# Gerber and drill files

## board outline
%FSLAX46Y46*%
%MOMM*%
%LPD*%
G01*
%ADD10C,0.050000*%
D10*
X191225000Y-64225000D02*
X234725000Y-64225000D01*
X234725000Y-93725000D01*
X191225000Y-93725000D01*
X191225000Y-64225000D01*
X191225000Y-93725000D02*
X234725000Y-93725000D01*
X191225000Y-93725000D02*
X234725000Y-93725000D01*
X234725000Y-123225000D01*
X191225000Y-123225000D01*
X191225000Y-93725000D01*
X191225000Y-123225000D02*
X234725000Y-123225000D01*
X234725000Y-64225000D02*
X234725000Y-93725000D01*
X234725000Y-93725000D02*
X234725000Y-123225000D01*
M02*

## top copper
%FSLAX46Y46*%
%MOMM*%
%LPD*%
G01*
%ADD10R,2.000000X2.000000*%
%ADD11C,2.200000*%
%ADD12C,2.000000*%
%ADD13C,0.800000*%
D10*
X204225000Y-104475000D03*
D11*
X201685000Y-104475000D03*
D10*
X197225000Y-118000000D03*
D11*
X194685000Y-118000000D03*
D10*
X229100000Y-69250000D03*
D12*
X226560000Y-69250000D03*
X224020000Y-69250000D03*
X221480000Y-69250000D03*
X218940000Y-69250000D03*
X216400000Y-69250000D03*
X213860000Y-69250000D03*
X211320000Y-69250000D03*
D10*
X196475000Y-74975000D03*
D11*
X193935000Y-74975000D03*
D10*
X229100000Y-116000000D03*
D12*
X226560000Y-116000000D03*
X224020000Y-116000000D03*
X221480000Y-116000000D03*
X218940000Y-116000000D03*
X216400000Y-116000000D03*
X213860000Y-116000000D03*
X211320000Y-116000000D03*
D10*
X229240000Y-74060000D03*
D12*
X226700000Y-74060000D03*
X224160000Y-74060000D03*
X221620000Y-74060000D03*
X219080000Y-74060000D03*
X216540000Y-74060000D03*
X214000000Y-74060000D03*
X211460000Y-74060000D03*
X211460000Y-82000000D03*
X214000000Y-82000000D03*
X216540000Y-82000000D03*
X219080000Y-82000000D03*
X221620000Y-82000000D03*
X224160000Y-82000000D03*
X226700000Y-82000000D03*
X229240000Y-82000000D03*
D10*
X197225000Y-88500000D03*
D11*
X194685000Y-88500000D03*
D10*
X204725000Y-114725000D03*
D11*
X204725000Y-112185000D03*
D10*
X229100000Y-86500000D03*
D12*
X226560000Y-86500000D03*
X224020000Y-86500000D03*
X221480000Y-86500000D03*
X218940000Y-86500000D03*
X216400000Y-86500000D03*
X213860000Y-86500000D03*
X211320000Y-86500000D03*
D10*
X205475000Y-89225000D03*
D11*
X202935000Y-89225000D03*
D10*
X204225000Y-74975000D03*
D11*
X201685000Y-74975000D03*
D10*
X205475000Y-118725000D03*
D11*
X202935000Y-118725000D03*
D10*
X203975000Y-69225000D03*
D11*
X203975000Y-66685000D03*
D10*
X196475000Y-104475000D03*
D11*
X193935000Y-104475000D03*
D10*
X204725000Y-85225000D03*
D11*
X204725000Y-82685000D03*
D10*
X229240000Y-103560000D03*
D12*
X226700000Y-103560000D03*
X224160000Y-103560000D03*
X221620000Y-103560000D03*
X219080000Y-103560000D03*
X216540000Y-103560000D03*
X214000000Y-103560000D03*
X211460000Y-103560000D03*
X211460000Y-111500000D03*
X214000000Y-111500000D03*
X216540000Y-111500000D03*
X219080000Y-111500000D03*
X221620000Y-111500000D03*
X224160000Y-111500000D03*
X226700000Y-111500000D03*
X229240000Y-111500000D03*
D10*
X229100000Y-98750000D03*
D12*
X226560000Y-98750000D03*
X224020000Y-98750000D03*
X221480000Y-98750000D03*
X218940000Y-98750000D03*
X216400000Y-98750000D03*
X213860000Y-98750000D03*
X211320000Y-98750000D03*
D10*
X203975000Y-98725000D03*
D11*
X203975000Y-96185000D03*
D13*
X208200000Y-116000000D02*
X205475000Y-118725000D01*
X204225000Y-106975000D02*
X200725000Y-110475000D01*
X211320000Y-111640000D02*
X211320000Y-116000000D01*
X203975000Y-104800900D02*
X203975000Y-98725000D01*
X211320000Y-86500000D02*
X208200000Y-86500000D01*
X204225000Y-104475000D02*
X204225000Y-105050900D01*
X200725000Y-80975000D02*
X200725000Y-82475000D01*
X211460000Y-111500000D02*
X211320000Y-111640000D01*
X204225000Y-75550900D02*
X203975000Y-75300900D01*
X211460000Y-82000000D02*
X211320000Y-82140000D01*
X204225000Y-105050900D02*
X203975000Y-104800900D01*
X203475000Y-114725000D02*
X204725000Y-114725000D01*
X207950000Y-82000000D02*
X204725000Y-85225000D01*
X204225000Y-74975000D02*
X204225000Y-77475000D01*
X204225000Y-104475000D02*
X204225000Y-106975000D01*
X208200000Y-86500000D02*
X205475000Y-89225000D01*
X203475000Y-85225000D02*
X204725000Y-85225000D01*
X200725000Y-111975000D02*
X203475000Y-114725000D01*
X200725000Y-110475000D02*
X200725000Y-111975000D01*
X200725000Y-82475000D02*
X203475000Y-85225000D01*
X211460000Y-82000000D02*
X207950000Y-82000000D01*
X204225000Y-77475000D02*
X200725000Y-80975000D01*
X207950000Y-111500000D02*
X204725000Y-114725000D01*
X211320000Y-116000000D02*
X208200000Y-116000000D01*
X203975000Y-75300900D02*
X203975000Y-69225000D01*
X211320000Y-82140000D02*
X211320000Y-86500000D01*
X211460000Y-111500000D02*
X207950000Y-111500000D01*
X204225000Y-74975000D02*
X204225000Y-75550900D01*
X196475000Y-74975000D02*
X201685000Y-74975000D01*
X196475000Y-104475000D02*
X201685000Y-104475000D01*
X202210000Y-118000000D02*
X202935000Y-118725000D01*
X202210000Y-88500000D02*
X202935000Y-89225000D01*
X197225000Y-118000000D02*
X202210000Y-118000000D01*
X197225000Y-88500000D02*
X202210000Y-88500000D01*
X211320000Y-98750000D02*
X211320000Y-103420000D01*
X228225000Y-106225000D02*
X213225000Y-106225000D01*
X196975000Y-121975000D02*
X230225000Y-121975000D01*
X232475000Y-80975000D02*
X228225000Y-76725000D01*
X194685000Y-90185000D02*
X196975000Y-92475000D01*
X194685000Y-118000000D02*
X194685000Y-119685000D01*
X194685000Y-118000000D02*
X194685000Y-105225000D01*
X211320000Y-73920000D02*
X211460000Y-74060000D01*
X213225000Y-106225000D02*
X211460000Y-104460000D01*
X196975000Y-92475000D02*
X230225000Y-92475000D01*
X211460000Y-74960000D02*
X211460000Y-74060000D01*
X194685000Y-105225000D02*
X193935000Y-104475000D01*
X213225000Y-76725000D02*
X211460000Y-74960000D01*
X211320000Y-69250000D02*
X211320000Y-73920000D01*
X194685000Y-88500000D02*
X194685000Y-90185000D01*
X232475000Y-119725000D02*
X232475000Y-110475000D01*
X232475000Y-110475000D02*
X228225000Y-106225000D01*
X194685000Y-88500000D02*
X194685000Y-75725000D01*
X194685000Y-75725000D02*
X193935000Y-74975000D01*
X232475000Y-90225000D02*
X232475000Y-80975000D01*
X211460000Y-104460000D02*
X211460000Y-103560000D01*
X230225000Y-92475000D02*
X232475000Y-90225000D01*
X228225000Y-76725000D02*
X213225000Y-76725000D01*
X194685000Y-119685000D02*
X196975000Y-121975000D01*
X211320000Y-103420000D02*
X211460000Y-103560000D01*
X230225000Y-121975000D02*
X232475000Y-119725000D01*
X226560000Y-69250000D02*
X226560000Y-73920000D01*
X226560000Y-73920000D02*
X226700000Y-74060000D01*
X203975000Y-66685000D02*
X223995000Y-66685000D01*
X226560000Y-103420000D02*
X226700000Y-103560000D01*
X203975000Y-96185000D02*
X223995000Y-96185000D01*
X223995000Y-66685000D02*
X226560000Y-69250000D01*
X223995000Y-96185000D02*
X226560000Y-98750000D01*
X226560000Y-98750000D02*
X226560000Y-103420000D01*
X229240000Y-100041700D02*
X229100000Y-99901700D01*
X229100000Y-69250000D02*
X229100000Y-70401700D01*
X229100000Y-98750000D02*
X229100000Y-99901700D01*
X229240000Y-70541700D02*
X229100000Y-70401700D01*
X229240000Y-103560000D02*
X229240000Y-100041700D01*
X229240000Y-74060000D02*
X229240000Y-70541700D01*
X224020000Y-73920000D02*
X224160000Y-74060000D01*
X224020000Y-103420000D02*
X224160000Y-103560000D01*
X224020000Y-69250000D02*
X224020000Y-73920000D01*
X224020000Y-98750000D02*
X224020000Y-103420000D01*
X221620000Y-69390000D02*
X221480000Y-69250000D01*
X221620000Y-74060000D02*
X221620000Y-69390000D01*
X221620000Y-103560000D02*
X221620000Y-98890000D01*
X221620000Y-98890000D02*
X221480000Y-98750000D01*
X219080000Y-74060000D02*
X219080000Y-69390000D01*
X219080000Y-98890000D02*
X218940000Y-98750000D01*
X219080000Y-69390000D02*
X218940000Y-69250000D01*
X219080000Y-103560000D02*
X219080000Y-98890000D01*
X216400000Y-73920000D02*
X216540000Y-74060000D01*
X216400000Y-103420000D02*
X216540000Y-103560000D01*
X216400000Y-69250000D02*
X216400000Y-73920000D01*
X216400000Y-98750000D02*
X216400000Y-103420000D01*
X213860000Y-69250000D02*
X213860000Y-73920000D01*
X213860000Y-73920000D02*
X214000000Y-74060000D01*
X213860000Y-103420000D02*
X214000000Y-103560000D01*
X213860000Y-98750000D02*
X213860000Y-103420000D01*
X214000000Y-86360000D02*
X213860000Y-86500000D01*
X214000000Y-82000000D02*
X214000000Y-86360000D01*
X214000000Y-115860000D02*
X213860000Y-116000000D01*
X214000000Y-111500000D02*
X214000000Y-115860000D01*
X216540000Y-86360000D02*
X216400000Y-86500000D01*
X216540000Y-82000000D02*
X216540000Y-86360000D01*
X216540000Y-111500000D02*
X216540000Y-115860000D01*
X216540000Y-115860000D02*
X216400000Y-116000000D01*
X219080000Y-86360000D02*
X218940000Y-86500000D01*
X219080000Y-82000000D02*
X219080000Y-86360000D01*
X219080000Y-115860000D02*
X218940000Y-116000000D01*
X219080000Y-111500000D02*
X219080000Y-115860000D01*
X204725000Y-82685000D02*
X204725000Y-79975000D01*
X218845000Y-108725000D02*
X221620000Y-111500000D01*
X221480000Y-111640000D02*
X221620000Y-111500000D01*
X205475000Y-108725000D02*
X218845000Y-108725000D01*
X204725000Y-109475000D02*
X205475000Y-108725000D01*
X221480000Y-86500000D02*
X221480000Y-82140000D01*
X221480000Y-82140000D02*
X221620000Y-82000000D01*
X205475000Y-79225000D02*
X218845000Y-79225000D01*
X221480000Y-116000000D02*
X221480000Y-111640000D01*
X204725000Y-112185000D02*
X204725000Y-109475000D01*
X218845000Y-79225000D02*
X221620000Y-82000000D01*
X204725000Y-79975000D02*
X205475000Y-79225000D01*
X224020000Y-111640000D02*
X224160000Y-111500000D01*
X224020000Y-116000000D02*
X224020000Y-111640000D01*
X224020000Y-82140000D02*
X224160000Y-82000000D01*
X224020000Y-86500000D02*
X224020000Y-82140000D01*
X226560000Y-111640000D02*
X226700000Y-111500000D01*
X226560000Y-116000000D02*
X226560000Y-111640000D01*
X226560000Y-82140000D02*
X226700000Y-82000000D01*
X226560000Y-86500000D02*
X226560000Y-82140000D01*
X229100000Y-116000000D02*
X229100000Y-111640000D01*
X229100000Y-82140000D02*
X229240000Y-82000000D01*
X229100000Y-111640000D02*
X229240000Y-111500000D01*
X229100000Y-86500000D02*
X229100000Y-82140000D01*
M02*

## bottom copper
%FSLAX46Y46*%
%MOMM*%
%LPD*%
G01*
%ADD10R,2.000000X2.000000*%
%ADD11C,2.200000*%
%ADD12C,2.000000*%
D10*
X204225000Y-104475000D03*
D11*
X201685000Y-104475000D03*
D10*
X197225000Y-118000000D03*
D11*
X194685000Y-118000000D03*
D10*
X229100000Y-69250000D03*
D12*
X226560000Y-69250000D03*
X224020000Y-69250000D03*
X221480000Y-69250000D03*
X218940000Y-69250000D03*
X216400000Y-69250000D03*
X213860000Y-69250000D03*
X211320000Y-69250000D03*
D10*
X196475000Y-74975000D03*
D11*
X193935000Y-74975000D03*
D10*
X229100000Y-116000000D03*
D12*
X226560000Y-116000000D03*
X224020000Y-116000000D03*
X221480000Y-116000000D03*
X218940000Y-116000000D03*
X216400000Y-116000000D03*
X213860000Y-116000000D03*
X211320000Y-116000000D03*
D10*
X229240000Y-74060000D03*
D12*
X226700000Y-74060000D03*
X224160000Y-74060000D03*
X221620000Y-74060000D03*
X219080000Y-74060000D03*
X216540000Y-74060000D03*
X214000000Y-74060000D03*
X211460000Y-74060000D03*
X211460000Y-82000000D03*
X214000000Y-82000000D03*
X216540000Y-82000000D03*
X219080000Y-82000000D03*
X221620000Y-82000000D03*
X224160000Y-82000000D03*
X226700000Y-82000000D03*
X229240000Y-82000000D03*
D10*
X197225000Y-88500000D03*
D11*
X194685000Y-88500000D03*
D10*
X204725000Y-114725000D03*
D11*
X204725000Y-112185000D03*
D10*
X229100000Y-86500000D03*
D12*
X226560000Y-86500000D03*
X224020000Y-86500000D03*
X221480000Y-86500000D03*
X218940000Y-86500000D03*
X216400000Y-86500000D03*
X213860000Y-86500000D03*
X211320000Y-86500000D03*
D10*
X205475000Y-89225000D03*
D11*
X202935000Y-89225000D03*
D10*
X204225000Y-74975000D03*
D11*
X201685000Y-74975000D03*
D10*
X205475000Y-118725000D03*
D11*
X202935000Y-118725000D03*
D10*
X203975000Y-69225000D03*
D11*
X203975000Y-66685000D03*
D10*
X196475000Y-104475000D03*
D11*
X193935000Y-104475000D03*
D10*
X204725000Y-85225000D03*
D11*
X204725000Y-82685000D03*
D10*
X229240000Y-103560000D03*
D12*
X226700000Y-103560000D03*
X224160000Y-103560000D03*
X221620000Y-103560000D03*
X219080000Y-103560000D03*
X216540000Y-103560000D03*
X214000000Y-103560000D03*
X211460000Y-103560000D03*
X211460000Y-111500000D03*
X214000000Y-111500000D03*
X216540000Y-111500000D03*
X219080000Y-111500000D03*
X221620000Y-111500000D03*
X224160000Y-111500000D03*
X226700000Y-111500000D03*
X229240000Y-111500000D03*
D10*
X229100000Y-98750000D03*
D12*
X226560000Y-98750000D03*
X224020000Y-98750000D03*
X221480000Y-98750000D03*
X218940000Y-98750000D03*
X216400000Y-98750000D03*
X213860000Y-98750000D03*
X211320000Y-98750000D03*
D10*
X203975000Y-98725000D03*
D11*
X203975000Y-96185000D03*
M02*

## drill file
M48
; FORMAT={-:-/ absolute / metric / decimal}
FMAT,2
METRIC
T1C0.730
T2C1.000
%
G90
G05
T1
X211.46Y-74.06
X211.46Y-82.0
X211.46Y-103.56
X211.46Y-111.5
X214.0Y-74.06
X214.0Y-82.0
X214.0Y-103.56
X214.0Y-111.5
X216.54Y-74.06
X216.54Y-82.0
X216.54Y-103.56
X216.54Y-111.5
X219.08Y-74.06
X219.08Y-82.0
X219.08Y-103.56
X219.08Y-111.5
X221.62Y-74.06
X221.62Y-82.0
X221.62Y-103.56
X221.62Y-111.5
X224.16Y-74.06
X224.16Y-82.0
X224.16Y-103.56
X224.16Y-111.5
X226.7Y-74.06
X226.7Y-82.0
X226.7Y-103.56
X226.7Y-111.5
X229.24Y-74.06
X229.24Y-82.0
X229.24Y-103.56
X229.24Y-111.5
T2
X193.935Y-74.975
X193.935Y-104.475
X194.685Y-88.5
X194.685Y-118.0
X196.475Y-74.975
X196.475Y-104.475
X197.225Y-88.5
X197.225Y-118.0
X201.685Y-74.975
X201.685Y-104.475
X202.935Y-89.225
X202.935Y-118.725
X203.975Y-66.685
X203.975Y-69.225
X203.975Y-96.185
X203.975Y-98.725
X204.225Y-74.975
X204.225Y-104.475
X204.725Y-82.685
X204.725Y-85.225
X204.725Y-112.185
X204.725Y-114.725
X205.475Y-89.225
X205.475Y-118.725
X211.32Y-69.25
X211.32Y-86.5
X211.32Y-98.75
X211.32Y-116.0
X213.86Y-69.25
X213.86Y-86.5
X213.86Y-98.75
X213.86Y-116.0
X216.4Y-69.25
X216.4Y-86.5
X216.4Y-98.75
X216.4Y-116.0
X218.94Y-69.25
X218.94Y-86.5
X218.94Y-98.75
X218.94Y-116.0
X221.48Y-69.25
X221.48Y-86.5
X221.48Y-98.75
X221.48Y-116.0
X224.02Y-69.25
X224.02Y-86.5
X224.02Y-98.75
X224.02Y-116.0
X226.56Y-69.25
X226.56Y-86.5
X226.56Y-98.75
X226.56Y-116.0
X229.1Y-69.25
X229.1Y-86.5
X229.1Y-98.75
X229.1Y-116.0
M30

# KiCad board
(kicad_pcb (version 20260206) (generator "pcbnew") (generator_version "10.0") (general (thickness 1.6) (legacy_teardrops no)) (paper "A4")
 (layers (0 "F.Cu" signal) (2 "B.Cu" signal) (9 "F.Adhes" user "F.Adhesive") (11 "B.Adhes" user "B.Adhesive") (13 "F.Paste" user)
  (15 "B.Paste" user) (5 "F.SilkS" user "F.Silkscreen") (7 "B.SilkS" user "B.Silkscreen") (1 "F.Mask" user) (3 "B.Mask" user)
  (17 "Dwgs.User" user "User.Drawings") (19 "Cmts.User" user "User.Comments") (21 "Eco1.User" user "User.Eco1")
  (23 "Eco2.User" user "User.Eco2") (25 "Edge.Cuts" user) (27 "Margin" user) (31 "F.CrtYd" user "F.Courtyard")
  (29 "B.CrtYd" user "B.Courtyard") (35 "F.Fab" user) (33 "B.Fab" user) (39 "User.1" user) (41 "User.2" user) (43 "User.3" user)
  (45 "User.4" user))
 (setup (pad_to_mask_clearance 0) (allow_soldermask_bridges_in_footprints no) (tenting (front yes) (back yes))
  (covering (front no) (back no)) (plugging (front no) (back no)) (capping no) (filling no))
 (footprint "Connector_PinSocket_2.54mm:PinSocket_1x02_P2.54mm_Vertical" (layer "F.Cu") (at 204.225 104.475 -90)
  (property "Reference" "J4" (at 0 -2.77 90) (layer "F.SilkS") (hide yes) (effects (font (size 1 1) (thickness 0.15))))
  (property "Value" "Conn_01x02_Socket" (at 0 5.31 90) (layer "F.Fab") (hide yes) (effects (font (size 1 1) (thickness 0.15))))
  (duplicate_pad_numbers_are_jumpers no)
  (pad "1" thru_hole rect (at 0 0 270) (size 2 2) (drill 1) (layers "*.Cu" "*.Mask") (remove_unused_layers no) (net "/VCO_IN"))
  (pad "2" thru_hole circle (at 0 2.54 270) (size 2.2 2.2) (drill 1) (layers "*.Cu" "*.Mask") (remove_unused_layers no)
   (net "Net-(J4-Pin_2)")))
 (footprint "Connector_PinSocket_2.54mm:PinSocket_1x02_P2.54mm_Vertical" (layer "F.Cu") (at 197.225 118 -90)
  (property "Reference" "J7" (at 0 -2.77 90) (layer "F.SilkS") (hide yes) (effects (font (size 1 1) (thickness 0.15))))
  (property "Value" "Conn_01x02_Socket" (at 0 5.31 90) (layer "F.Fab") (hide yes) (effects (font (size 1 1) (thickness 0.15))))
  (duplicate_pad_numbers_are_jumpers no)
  (pad "1" thru_hole rect (at 0 0 270) (size 2 2) (drill 1) (layers "*.Cu" "*.Mask") (remove_unused_layers no) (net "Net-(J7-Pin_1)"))
  (pad "2" thru_hole circle (at 0 2.54 270) (size 2.2 2.2) (drill 1) (layers "*.Cu" "*.Mask") (remove_unused_layers no) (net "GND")))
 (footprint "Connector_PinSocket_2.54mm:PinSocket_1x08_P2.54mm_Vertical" (layer "F.Cu") (at 229.1 69.25 -90)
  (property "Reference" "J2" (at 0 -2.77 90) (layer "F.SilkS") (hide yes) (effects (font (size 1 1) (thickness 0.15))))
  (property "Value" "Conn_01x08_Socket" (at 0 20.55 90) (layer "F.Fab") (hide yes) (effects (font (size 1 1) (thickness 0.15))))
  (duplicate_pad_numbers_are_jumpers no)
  (pad "1" thru_hole rect (at 0 0 270) (size 2 2) (drill 1) (layers "*.Cu" "*.Mask") (remove_unused_layers no)
   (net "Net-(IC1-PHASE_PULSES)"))
  (pad "2" thru_hole circle (at 0 2.54 270) (size 2 2) (drill 1) (layers "*.Cu" "*.Mask") (remove_unused_layers no) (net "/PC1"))
  (pad "3" thru_hole circle (at 0 5.08 270) (size 2 2) (drill 1) (layers "*.Cu" "*.Mask") (remove_unused_layers no)
   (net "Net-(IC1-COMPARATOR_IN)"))
  (pad "4" thru_hole circle (at 0 7.62 270) (size 2 2) (drill 1) (layers "*.Cu" "*.Mask") (remove_unused_layers no)
   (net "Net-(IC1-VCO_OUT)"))
  (pad "5" thru_hole circle (at 0 10.16 270) (size 2 2) (drill 1) (layers "*.Cu" "*.Mask") (remove_unused_layers no)
   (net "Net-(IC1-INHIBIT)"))
  (pad "6" thru_hole circle (at 0 12.7 270) (size 2 2) (drill 1) (layers "*.Cu" "*.Mask") (remove_unused_layers no) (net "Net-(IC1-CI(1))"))
  (pad "7" thru_hole circle (at 0 15.24 270) (size 2 2) (drill 1) (layers "*.Cu" "*.Mask") (remove_unused_layers no) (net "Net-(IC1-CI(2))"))
  (pad "8" thru_hole circle (at 0 17.78 270) (size 2 2) (drill 1) (layers "*.Cu" "*.Mask") (remove_unused_layers no) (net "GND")))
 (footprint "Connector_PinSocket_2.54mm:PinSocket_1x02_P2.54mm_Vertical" (layer "F.Cu") (at 196.475 74.975 -90)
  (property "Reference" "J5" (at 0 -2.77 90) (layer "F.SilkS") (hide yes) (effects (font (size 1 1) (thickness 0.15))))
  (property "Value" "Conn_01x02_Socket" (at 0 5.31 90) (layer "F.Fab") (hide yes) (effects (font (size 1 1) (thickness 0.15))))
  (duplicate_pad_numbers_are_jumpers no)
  (pad "1" thru_hole rect (at 0 0 270) (size 2 2) (drill 1) (layers "*.Cu" "*.Mask") (remove_unused_layers no) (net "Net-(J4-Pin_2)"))
  (pad "2" thru_hole circle (at 0 2.54 270) (size 2.2 2.2) (drill 1) (layers "*.Cu" "*.Mask") (remove_unused_layers no) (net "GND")))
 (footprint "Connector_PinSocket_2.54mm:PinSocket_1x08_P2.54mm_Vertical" (layer "F.Cu") (at 229.1 116 -90)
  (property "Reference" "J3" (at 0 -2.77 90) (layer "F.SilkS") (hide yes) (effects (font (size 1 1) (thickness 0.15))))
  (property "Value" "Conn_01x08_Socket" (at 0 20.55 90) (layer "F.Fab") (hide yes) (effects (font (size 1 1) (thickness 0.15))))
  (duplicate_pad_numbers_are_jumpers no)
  (pad "1" thru_hole rect (at 0 0 270) (size 2 2) (drill 1) (layers "*.Cu" "*.Mask") (remove_unused_layers no) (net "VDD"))
  (pad "2" thru_hole circle (at 0 2.54 270) (size 2 2) (drill 1) (layers "*.Cu" "*.Mask") (remove_unused_layers no) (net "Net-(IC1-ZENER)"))
  (pad "3" thru_hole circle (at 0 5.08 270) (size 2 2) (drill 1) (layers "*.Cu" "*.Mask") (remove_unused_layers no)
   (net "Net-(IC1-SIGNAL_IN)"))
  (pad "4" thru_hole circle (at 0 7.62 270) (size 2 2) (drill 1) (layers "*.Cu" "*.Mask") (remove_unused_layers no) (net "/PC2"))
  (pad "5" thru_hole circle (at 0 10.16 270) (size 2 2) (drill 1) (layers "*.Cu" "*.Mask") (remove_unused_layers no)
   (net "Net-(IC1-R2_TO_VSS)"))
  (pad "6" thru_hole circle (at 0 12.7 270) (size 2 2) (drill 1) (layers "*.Cu" "*.Mask") (remove_unused_layers no)
   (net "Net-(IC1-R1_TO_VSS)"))
  (pad "7" thru_hole circle (at 0 15.24 270) (size 2 2) (drill 1) (layers "*.Cu" "*.Mask") (remove_unused_layers no)
   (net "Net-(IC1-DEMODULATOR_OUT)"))
  (pad "8" thru_hole circle (at 0 17.78 270) (size 2 2) (drill 1) (layers "*.Cu" "*.Mask") (remove_unused_layers no) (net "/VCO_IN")))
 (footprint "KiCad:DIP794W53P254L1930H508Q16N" (layer "F.Cu") (at 220.35 78.03 -90)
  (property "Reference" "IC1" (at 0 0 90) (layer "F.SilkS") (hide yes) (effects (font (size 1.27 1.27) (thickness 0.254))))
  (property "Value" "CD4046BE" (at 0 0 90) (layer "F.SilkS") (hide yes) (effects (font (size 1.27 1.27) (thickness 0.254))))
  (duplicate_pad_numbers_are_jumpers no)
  (pad "1" thru_hole rect (at -3.97 -8.89 270) (size 2 2) (drill 0.73) (layers "*.Cu" "*.Mask") (remove_unused_layers no)
   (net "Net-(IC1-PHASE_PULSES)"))
  (pad "2" thru_hole circle (at -3.97 -6.35 270) (size 2 2) (drill 0.73) (layers "*.Cu" "*.Mask") (remove_unused_layers no) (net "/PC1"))
  (pad "3" thru_hole circle (at -3.97 -3.81 270) (size 2 2) (drill 0.73) (layers "*.Cu" "*.Mask") (remove_unused_layers no)
   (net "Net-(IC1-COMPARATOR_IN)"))
  (pad "4" thru_hole circle (at -3.97 -1.27 270) (size 2 2) (drill 0.73) (layers "*.Cu" "*.Mask") (remove_unused_layers no)
   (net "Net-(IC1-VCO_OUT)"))
  (pad "5" thru_hole circle (at -3.97 1.27 270) (size 2 2) (drill 0.73) (layers "*.Cu" "*.Mask") (remove_unused_layers no)
   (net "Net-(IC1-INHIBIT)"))
  (pad "6" thru_hole circle (at -3.97 3.81 270) (size 2 2) (drill 0.73) (layers "*.Cu" "*.Mask") (remove_unused_layers no)
   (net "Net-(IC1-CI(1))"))
  (pad "7" thru_hole circle (at -3.97 6.35 270) (size 2 2) (drill 0.73) (layers "*.Cu" "*.Mask") (remove_unused_layers no)
   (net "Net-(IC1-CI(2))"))
  (pad "8" thru_hole circle (at -3.97 8.89 270) (size 2 2) (drill 0.73) (layers "*.Cu" "*.Mask") (remove_unused_layers no) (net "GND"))
  (pad "9" thru_hole circle (at 3.97 8.89 270) (size 2 2) (drill 0.73) (layers "*.Cu" "*.Mask") (remove_unused_layers no) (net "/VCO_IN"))
  (pad "10" thru_hole circle (at 3.97 6.35 270) (size 2 2) (drill 0.73) (layers "*.Cu" "*.Mask") (remove_unused_layers no)
   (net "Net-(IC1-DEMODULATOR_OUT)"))
  (pad "11" thru_hole circle (at 3.97 3.81 270) (size 2 2) (drill 0.73) (layers "*.Cu" "*.Mask") (remove_unused_layers no)
   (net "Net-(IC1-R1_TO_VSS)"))
  (pad "12" thru_hole circle (at 3.97 1.27 270) (size 2 2) (drill 0.73) (layers "*.Cu" "*.Mask") (remove_unused_layers no)
   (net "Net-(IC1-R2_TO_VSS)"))
  (pad "13" thru_hole circle (at 3.97 -1.27 270) (size 2 2) (drill 0.73) (layers "*.Cu" "*.Mask") (remove_unused_layers no) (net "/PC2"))
  (pad "14" thru_hole circle (at 3.97 -3.81 270) (size 2 2) (drill 0.73) (layers "*.Cu" "*.Mask") (remove_unused_layers no)
   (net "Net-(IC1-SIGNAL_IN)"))
  (pad "15" thru_hole circle (at 3.97 -6.35 270) (size 2 2) (drill 0.73) (layers "*.Cu" "*.Mask") (remove_unused_layers no)
   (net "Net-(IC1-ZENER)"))
  (pad "16" thru_hole circle (at 3.97 -8.89 270) (size 2 2) (drill 0.73) (layers "*.Cu" "*.Mask") (remove_unused_layers no) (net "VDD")))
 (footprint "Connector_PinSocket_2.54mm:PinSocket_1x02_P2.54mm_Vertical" (layer "F.Cu") (at 197.225 88.5 -90)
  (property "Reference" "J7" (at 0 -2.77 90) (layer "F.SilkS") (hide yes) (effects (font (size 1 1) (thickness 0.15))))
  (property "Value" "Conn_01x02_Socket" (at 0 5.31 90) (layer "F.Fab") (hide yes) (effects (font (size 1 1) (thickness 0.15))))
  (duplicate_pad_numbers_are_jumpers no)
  (pad "1" thru_hole rect (at 0 0 270) (size 2 2) (drill 1) (layers "*.Cu" "*.Mask") (remove_unused_layers no) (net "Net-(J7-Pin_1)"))
  (pad "2" thru_hole circle (at 0 2.54 270) (size 2.2 2.2) (drill 1) (layers "*.Cu" "*.Mask") (remove_unused_layers no) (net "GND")))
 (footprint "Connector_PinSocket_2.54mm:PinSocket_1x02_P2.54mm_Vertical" (layer "F.Cu") (at 204.725 114.725 180)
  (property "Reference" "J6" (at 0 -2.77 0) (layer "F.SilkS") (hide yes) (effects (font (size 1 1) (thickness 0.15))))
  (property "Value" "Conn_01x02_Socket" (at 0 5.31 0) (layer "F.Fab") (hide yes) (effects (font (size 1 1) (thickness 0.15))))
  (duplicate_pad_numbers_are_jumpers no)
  (pad "1" thru_hole rect (at 0 0 180) (size 2 2) (drill 1) (layers "*.Cu" "*.Mask") (remove_unused_layers no) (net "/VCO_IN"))
  (pad "2" thru_hole circle (at 0 2.54 180) (size 2.2 2.2) (drill 1) (layers "*.Cu" "*.Mask") (remove_unused_layers no) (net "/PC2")))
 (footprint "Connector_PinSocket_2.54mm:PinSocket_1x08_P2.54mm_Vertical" (layer "F.Cu") (at 229.1 86.5 -90)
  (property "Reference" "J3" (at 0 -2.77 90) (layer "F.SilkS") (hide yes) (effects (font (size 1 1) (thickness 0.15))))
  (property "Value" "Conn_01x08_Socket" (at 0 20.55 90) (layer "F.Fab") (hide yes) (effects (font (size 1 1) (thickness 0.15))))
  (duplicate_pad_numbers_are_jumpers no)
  (pad "1" thru_hole rect (at 0 0 270) (size 2 2) (drill 1) (layers "*.Cu" "*.Mask") (remove_unused_layers no) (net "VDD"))
  (pad "2" thru_hole circle (at 0 2.54 270) (size 2 2) (drill 1) (layers "*.Cu" "*.Mask") (remove_unused_layers no) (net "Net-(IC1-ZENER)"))
  (pad "3" thru_hole circle (at 0 5.08 270) (size 2 2) (drill 1) (layers "*.Cu" "*.Mask") (remove_unused_layers no)
   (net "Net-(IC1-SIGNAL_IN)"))
  (pad "4" thru_hole circle (at 0 7.62 270) (size 2 2) (drill 1) (layers "*.Cu" "*.Mask") (remove_unused_layers no) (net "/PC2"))
  (pad "5" thru_hole circle (at 0 10.16 270) (size 2 2) (drill 1) (layers "*.Cu" "*.Mask") (remove_unused_layers no)
   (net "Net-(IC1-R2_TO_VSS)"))
  (pad "6" thru_hole circle (at 0 12.7 270) (size 2 2) (drill 1) (layers "*.Cu" "*.Mask") (remove_unused_layers no)
   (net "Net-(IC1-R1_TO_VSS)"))
  (pad "7" thru_hole circle (at 0 15.24 270) (size 2 2) (drill 1) (layers "*.Cu" "*.Mask") (remove_unused_layers no)
   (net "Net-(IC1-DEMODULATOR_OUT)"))
  (pad "8" thru_hole circle (at 0 17.78 270) (size 2 2) (drill 1) (layers "*.Cu" "*.Mask") (remove_unused_layers no) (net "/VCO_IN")))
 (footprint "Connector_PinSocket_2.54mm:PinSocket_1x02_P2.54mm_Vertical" (layer "F.Cu") (at 205.475 89.225 -90)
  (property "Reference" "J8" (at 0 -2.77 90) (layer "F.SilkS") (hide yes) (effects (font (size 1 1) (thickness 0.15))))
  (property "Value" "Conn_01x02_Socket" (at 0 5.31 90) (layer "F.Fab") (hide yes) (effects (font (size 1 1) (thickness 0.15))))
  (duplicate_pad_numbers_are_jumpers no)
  (pad "1" thru_hole rect (at 0 0 270) (size 2 2) (drill 1) (layers "*.Cu" "*.Mask") (remove_unused_layers no) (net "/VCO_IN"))
  (pad "2" thru_hole circle (at 0 2.54 270) (size 2.2 2.2) (drill 1) (layers "*.Cu" "*.Mask") (remove_unused_layers no)
   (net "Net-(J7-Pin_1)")))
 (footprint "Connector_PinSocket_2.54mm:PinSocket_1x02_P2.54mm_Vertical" (layer "F.Cu") (at 204.225 74.975 -90)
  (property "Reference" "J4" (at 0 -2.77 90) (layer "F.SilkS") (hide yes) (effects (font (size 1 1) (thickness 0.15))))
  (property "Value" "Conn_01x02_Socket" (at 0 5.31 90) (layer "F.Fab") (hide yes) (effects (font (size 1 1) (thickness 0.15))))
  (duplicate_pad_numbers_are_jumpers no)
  (pad "1" thru_hole rect (at 0 0 270) (size 2 2) (drill 1) (layers "*.Cu" "*.Mask") (remove_unused_layers no) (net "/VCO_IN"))
  (pad "2" thru_hole circle (at 0 2.54 270) (size 2.2 2.2) (drill 1) (layers "*.Cu" "*.Mask") (remove_unused_layers no)
   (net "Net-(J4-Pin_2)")))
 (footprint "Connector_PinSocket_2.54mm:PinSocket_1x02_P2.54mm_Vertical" (layer "F.Cu") (at 205.475 118.725 -90)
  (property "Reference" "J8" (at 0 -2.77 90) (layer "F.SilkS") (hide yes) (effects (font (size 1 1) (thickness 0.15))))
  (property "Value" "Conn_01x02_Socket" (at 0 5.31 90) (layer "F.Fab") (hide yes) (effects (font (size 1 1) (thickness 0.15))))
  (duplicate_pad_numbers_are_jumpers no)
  (pad "1" thru_hole rect (at 0 0 270) (size 2 2) (drill 1) (layers "*.Cu" "*.Mask") (remove_unused_layers no) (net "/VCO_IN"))
  (pad "2" thru_hole circle (at 0 2.54 270) (size 2.2 2.2) (drill 1) (layers "*.Cu" "*.Mask") (remove_unused_layers no)
   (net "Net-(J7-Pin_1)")))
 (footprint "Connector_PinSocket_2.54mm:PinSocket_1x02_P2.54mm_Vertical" (layer "F.Cu") (at 203.975 69.225 180)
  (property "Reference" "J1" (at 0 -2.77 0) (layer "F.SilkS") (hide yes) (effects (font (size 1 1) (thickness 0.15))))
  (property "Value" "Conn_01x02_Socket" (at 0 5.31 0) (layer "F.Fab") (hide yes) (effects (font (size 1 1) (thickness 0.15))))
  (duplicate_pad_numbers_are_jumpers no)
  (pad "1" thru_hole rect (at 0 0 180) (size 2 2) (drill 1) (layers "*.Cu" "*.Mask") (remove_unused_layers no) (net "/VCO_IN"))
  (pad "2" thru_hole circle (at 0 2.54 180) (size 2.2 2.2) (drill 1) (layers "*.Cu" "*.Mask") (remove_unused_layers no) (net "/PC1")))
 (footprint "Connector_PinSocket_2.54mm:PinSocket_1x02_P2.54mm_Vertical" (layer "F.Cu") (at 196.475 104.475 -90)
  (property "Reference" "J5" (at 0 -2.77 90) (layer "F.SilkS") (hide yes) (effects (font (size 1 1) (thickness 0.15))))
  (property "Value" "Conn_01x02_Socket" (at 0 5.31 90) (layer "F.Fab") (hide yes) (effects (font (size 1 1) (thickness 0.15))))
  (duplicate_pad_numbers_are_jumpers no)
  (pad "1" thru_hole rect (at 0 0 270) (size 2 2) (drill 1) (layers "*.Cu" "*.Mask") (remove_unused_layers no) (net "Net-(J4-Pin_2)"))
  (pad "2" thru_hole circle (at 0 2.54 270) (size 2.2 2.2) (drill 1) (layers "*.Cu" "*.Mask") (remove_unused_layers no) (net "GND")))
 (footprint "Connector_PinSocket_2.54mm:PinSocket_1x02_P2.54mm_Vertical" (layer "F.Cu") (at 204.725 85.225 180)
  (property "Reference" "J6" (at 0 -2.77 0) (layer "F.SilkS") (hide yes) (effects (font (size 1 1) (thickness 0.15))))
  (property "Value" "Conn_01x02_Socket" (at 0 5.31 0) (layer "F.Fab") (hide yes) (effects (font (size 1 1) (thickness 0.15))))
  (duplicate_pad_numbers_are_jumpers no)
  (pad "1" thru_hole rect (at 0 0 180) (size 2 2) (drill 1) (layers "*.Cu" "*.Mask") (remove_unused_layers no) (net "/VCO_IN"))
  (pad "2" thru_hole circle (at 0 2.54 180) (size 2.2 2.2) (drill 1) (layers "*.Cu" "*.Mask") (remove_unused_layers no) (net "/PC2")))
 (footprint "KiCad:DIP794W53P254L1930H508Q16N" (layer "F.Cu") (at 220.35 107.53 -90)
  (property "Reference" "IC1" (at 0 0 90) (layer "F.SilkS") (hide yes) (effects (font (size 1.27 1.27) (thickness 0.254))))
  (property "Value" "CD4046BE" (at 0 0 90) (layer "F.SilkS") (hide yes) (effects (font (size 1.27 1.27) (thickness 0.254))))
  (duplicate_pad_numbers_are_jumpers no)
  (pad "1" thru_hole rect (at -3.97 -8.89 270) (size 2 2) (drill 0.73) (layers "*.Cu" "*.Mask") (remove_unused_layers no)
   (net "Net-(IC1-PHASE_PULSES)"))
  (pad "2" thru_hole circle (at -3.97 -6.35 270) (size 2 2) (drill 0.73) (layers "*.Cu" "*.Mask") (remove_unused_layers no) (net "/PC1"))
  (pad "3" thru_hole circle (at -3.97 -3.81 270) (size 2 2) (drill 0.73) (layers "*.Cu" "*.Mask") (remove_unused_layers no)
   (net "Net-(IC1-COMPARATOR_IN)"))
  (pad "4" thru_hole circle (at -3.97 -1.27 270) (size 2 2) (drill 0.73) (layers "*.Cu" "*.Mask") (remove_unused_layers no)
   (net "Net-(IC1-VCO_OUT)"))
  (pad "5" thru_hole circle (at -3.97 1.27 270) (size 2 2) (drill 0.73) (layers "*.Cu" "*.Mask") (remove_unused_layers no)
   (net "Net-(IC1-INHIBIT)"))
  (pad "6" thru_hole circle (at -3.97 3.81 270) (size 2 2) (drill 0.73) (layers "*.Cu" "*.Mask") (remove_unused_layers no)
   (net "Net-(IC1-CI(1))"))
  (pad "7" thru_hole circle (at -3.97 6.35 270) (size 2 2) (drill 0.73) (layers "*.Cu" "*.Mask") (remove_unused_layers no)
   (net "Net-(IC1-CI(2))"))
  (pad "8" thru_hole circle (at -3.97 8.89 270) (size 2 2) (drill 0.73) (layers "*.Cu" "*.Mask") (remove_unused_layers no) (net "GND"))
  (pad "9" thru_hole circle (at 3.97 8.89 270) (size 2 2) (drill 0.73) (layers "*.Cu" "*.Mask") (remove_unused_layers no) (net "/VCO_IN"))
  (pad "10" thru_hole circle (at 3.97 6.35 270) (size 2 2) (drill 0.73) (layers "*.Cu" "*.Mask") (remove_unused_layers no)
   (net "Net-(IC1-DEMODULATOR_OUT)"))
  (pad "11" thru_hole circle (at 3.97 3.81 270) (size 2 2) (drill 0.73) (layers "*.Cu" "*.Mask") (remove_unused_layers no)
   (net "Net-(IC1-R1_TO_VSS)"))
  (pad "12" thru_hole circle (at 3.97 1.27 270) (size 2 2) (drill 0.73) (layers "*.Cu" "*.Mask") (remove_unused_layers no)
   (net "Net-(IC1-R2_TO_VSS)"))
  (pad "13" thru_hole circle (at 3.97 -1.27 270) (size 2 2) (drill 0.73) (layers "*.Cu" "*.Mask") (remove_unused_layers no) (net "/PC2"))
  (pad "14" thru_hole circle (at 3.97 -3.81 270) (size 2 2) (drill 0.73) (layers "*.Cu" "*.Mask") (remove_unused_layers no)
   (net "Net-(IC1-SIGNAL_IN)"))
  (pad "15" thru_hole circle (at 3.97 -6.35 270) (size 2 2) (drill 0.73) (layers "*.Cu" "*.Mask") (remove_unused_layers no)
   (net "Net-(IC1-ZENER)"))
  (pad "16" thru_hole circle (at 3.97 -8.89 270) (size 2 2) (drill 0.73) (layers "*.Cu" "*.Mask") (remove_unused_layers no) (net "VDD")))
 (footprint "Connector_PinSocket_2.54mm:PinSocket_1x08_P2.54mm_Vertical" (layer "F.Cu") (at 229.1 98.75 -90)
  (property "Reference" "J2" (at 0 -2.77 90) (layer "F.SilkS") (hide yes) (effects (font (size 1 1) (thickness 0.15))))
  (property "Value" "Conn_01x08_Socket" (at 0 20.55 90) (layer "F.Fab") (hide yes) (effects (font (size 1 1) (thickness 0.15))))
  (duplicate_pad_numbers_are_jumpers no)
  (pad "1" thru_hole rect (at 0 0 270) (size 2 2) (drill 1) (layers "*.Cu" "*.Mask") (remove_unused_layers no)
   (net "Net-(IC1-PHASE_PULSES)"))
  (pad "2" thru_hole circle (at 0 2.54 270) (size 2 2) (drill 1) (layers "*.Cu" "*.Mask") (remove_unused_layers no) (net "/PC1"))
  (pad "3" thru_hole circle (at 0 5.08 270) (size 2 2) (drill 1) (layers "*.Cu" "*.Mask") (remove_unused_layers no)
   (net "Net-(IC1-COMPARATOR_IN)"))
  (pad "4" thru_hole circle (at 0 7.62 270) (size 2 2) (drill 1) (layers "*.Cu" "*.Mask") (remove_unused_layers no)
   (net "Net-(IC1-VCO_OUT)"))
  (pad "5" thru_hole circle (at 0 10.16 270) (size 2 2) (drill 1) (layers "*.Cu" "*.Mask") (remove_unused_layers no)
   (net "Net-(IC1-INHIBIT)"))
  (pad "6" thru_hole circle (at 0 12.7 270) (size 2 2) (drill 1) (layers "*.Cu" "*.Mask") (remove_unused_layers no) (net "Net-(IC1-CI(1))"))
  (pad "7" thru_hole circle (at 0 15.24 270) (size 2 2) (drill 1) (layers "*.Cu" "*.Mask") (remove_unused_layers no) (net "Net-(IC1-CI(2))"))
  (pad "8" thru_hole circle (at 0 17.78 270) (size 2 2) (drill 1) (layers "*.Cu" "*.Mask") (remove_unused_layers no) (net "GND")))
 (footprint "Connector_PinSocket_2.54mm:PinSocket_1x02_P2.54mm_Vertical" (layer "F.Cu") (at 203.975 98.725 180)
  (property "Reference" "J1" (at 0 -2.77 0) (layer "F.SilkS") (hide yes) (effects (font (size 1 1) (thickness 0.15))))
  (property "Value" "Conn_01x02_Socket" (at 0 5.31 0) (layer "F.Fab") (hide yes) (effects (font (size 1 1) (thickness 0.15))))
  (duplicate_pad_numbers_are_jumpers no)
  (pad "1" thru_hole rect (at 0 0 180) (size 2 2) (drill 1) (layers "*.Cu" "*.Mask") (remove_unused_layers no) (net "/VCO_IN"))
  (pad "2" thru_hole circle (at 0 2.54 180) (size 2.2 2.2) (drill 1) (layers "*.Cu" "*.Mask") (remove_unused_layers no) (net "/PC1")))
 (gr_rect (start 191.225 64.225) (end 234.725 93.725) (stroke (width 0.05) (type default)) (fill no) (layer "Edge.Cuts"))
 (gr_line (start 191.225 93.725) (end 234.725 93.725) (stroke (width 0.05) (type default)) (layer "Edge.Cuts"))
 (gr_rect (start 191.225 93.725) (end 234.725 123.225) (stroke (width 0.05) (type default)) (fill no) (layer "Edge.Cuts"))
 (gr_line (start 191.225 123.225) (end 234.725 123.225) (stroke (width 0.05) (type default)) (layer "Edge.Cuts"))
 (gr_line (start 234.725 64.225) (end 234.725 93.725) (stroke (width 0.05) (type default)) (layer "Edge.Cuts"))
 (gr_line (start 234.725 93.725) (end 234.725 123.225) (stroke (width 0.05) (type default)) (layer "Edge.Cuts"))
 (segment (start 208.2 116) (end 205.475 118.725) (width 0.8) (layer "F.Cu") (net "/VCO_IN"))
 (segment (start 204.225 106.975) (end 200.725 110.475) (width 0.8) (layer "F.Cu") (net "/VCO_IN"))
 (segment (start 211.32 111.64) (end 211.32 116) (width 0.8) (layer "F.Cu") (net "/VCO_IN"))
 (segment (start 203.975 104.8009) (end 203.975 98.725) (width 0.8) (layer "F.Cu") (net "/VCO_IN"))
 (segment (start 211.32 86.5) (end 208.2 86.5) (width 0.8) (layer "F.Cu") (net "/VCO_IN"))
 (segment (start 204.225 104.475) (end 204.225 105.0509) (width 0.8) (layer "F.Cu") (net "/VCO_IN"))
 (segment (start 200.725 80.975) (end 200.725 82.475) (width 0.8) (layer "F.Cu") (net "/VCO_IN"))
 (segment (start 211.46 111.5) (end 211.32 111.64) (width 0.8) (layer "F.Cu") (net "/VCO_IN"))
 (segment (start 204.225 75.5509) (end 203.975 75.3009) (width 0.8) (layer "F.Cu") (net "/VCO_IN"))
 (segment (start 211.46 82) (end 211.32 82.14) (width 0.8) (layer "F.Cu") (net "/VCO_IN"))
 (segment (start 204.225 105.0509) (end 203.975 104.8009) (width 0.8) (layer "F.Cu") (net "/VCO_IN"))
 (segment (start 203.475 114.725) (end 204.725 114.725) (width 0.8) (layer "F.Cu") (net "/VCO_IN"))
 (segment (start 207.95 82) (end 204.725 85.225) (width 0.8) (layer "F.Cu") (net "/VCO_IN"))
 (segment (start 204.225 74.975) (end 204.225 77.475) (width 0.8) (layer "F.Cu") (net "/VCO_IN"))
 (segment (start 204.225 104.475) (end 204.225 106.975) (width 0.8) (layer "F.Cu") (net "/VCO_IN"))
 (segment (start 208.2 86.5) (end 205.475 89.225) (width 0.8) (layer "F.Cu") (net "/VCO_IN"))
 (segment (start 203.475 85.225) (end 204.725 85.225) (width 0.8) (layer "F.Cu") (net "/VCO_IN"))
 (segment (start 200.725 111.975) (end 203.475 114.725) (width 0.8) (layer "F.Cu") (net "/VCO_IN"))
 (segment (start 200.725 110.475) (end 200.725 111.975) (width 0.8) (layer "F.Cu") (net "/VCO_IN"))
 (segment (start 200.725 82.475) (end 203.475 85.225) (width 0.8) (layer "F.Cu") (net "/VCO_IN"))
 (segment (start 211.46 82) (end 207.95 82) (width 0.8) (layer "F.Cu") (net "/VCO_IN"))
 (segment (start 204.225 77.475) (end 200.725 80.975) (width 0.8) (layer "F.Cu") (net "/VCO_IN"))
 (segment (start 207.95 111.5) (end 204.725 114.725) (width 0.8) (layer "F.Cu") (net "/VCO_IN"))
 (segment (start 211.32 116) (end 208.2 116) (width 0.8) (layer "F.Cu") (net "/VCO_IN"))
 (segment (start 203.975 75.3009) (end 203.975 69.225) (width 0.8) (layer "F.Cu") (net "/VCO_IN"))
 (segment (start 211.32 82.14) (end 211.32 86.5) (width 0.8) (layer "F.Cu") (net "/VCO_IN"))
 (segment (start 211.46 111.5) (end 207.95 111.5) (width 0.8) (layer "F.Cu") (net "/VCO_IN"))
 (segment (start 204.225 74.975) (end 204.225 75.5509) (width 0.8) (layer "F.Cu") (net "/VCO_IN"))
 (segment (start 196.475 74.975) (end 201.685 74.975) (width 0.8) (layer "F.Cu") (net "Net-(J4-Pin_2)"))
 (segment (start 196.475 104.475) (end 201.685 104.475) (width 0.8) (layer "F.Cu") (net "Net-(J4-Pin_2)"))
 (segment (start 202.21 118) (end 202.935 118.725) (width 0.8) (layer "F.Cu") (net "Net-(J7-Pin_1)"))
 (segment (start 202.21 88.5) (end 202.935 89.225) (width 0.8) (layer "F.Cu") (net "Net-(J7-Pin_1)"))
 (segment (start 197.225 118) (end 202.21 118) (width 0.8) (layer "F.Cu") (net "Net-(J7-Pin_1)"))
 (segment (start 197.225 88.5) (end 202.21 88.5) (width 0.8) (layer "F.Cu") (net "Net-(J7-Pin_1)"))
 (segment (start 211.32 98.75) (end 211.32 103.42) (width 0.8) (layer "F.Cu") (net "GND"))
 (segment (start 228.225 106.225) (end 213.225 106.225) (width 0.8) (layer "F.Cu") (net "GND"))
 (segment (start 196.975 121.975) (end 230.225 121.975) (width 0.8) (layer "F.Cu") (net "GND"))
 (segment (start 232.475 80.975) (end 228.225 76.725) (width 0.8) (layer "F.Cu") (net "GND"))
 (segment (start 194.685 90.185) (end 196.975 92.475) (width 0.8) (layer "F.Cu") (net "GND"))
 (segment (start 194.685 118) (end 194.685 119.685) (width 0.8) (layer "F.Cu") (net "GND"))
 (segment (start 194.685 118) (end 194.685 105.225) (width 0.8) (layer "F.Cu") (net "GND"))
 (segment (start 211.32 73.92) (end 211.46 74.06) (width 0.8) (layer "F.Cu") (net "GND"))
 (segment (start 213.225 106.225) (end 211.46 104.46) (width 0.8) (layer "F.Cu") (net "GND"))
 (segment (start 196.975 92.475) (end 230.225 92.475) (width 0.8) (layer "F.Cu") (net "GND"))
 (segment (start 211.46 74.96) (end 211.46 74.06) (width 0.8) (layer "F.Cu") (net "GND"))
 (segment (start 194.685 105.225) (end 193.935 104.475) (width 0.8) (layer "F.Cu") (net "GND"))
 (segment (start 213.225 76.725) (end 211.46 74.96) (width 0.8) (layer "F.Cu") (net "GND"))
 (segment (start 211.32 69.25) (end 211.32 73.92) (width 0.8) (layer "F.Cu") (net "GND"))
 (segment (start 194.685 88.5) (end 194.685 90.185) (width 0.8) (layer "F.Cu") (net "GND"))
 (segment (start 232.475 119.725) (end 232.475 110.475) (width 0.8) (layer "F.Cu") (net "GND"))
 (segment (start 232.475 110.475) (end 228.225 106.225) (width 0.8) (layer "F.Cu") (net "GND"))
 (segment (start 194.685 88.5) (end 194.685 75.725) (width 0.8) (layer "F.Cu") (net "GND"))
 (segment (start 194.685 75.725) (end 193.935 74.975) (width 0.8) (layer "F.Cu") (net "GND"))
 (segment (start 232.475 90.225) (end 232.475 80.975) (width 0.8) (layer "F.Cu") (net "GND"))
 (segment (start 211.46 104.46) (end 211.46 103.56) (width 0.8) (layer "F.Cu") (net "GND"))
 (segment (start 230.225 92.475) (end 232.475 90.225) (width 0.8) (layer "F.Cu") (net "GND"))
 (segment (start 228.225 76.725) (end 213.225 76.725) (width 0.8) (layer "F.Cu") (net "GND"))
 (segment (start 194.685 119.685) (end 196.975 121.975) (width 0.8) (layer "F.Cu") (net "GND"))
 (segment (start 211.32 103.42) (end 211.46 103.56) (width 0.8) (layer "F.Cu") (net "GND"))
 (segment (start 230.225 121.975) (end 232.475 119.725) (width 0.8) (layer "F.Cu") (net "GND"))
 (segment (start 226.56 69.25) (end 226.56 73.92) (width 0.8) (layer "F.Cu") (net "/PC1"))
 (segment (start 226.56 73.92) (end 226.7 74.06) (width 0.8) (layer "F.Cu") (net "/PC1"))
 (segment (start 203.975 66.685) (end 223.995 66.685) (width 0.8) (layer "F.Cu") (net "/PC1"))
 (segment (start 226.56 103.42) (end 226.7 103.56) (width 0.8) (layer "F.Cu") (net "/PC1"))
 (segment (start 203.975 96.185) (end 223.995 96.185) (width 0.8) (layer "F.Cu") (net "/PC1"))
 (segment (start 223.995 66.685) (end 226.56 69.25) (width 0.8) (layer "F.Cu") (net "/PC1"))
 (segment (start 223.995 96.185) (end 226.56 98.75) (width 0.8) (layer "F.Cu") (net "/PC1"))
 (segment (start 226.56 98.75) (end 226.56 103.42) (width 0.8) (layer "F.Cu") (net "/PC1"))
 (segment (start 229.24 100.0417) (end 229.1 99.9017) (width 0.8) (layer "F.Cu") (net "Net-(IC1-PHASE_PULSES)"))
 (segment (start 229.1 69.25) (end 229.1 70.4017) (width 0.8) (layer "F.Cu") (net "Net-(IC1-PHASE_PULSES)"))
 (segment (start 229.1 98.75) (end 229.1 99.9017) (width 0.8) (layer "F.Cu") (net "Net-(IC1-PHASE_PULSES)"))
 (segment (start 229.24 70.5417) (end 229.1 70.4017) (width 0.8) (layer "F.Cu") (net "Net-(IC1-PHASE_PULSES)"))
 (segment (start 229.24 103.56) (end 229.24 100.0417) (width 0.8) (layer "F.Cu") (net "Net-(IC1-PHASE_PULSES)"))
 (segment (start 229.24 74.06) (end 229.24 70.5417) (width 0.8) (layer "F.Cu") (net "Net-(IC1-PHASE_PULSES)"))
 (segment (start 224.02 73.92) (end 224.16 74.06) (width 0.8) (layer "F.Cu") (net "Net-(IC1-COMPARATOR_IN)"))
 (segment (start 224.02 103.42) (end 224.16 103.56) (width 0.8) (layer "F.Cu") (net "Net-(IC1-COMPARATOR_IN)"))
 (segment (start 224.02 69.25) (end 224.02 73.92) (width 0.8) (layer "F.Cu") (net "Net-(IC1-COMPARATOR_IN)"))
 (segment (start 224.02 98.75) (end 224.02 103.42) (width 0.8) (layer "F.Cu") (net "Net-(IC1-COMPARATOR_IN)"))
 (segment (start 221.62 69.39) (end 221.48 69.25) (width 0.8) (layer "F.Cu") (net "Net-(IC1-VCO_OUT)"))
 (segment (start 221.62 74.06) (end 221.62 69.39) (width 0.8) (layer "F.Cu") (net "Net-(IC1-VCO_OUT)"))
 (segment (start 221.62 103.56) (end 221.62 98.89) (width 0.8) (layer "F.Cu") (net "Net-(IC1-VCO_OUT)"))
 (segment (start 221.62 98.89) (end 221.48 98.75) (width 0.8) (layer "F.Cu") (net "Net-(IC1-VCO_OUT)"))
 (segment (start 219.08 74.06) (end 219.08 69.39) (width 0.8) (layer "F.Cu") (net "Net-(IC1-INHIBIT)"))
 (segment (start 219.08 98.89) (end 218.94 98.75) (width 0.8) (layer "F.Cu") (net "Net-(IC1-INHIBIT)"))
 (segment (start 219.08 69.39) (end 218.94 69.25) (width 0.8) (layer "F.Cu") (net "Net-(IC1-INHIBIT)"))
 (segment (start 219.08 103.56) (end 219.08 98.89) (width 0.8) (layer "F.Cu") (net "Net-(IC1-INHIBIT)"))
 (segment (start 216.4 73.92) (end 216.54 74.06) (width 0.8) (layer "F.Cu") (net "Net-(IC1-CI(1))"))
 (segment (start 216.4 103.42) (end 216.54 103.56) (width 0.8) (layer "F.Cu") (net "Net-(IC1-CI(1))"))
 (segment (start 216.4 69.25) (end 216.4 73.92) (width 0.8) (layer "F.Cu") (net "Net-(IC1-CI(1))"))
 (segment (start 216.4 98.75) (end 216.4 103.42) (width 0.8) (layer "F.Cu") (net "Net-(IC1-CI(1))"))
 (segment (start 213.86 69.25) (end 213.86 73.92) (width 0.8) (layer "F.Cu") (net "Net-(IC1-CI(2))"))
 (segment (start 213.86 73.92) (end 214 74.06) (width 0.8) (layer "F.Cu") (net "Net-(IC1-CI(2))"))
 (segment (start 213.86 103.42) (end 214 103.56) (width 0.8) (layer "F.Cu") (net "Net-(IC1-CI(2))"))
 (segment (start 213.86 98.75) (end 213.86 103.42) (width 0.8) (layer "F.Cu") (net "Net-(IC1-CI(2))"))
 (segment (start 214 86.36) (end 213.86 86.5) (width 0.8) (layer "F.Cu") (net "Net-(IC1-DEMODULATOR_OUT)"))
 (segment (start 214 82) (end 214 86.36) (width 0.8) (layer "F.Cu") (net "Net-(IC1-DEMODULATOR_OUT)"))
 (segment (start 214 115.86) (end 213.86 116) (width 0.8) (layer "F.Cu") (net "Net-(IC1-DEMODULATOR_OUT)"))
 (segment (start 214 111.5) (end 214 115.86) (width 0.8) (layer "F.Cu") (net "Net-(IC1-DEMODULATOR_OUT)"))
 (segment (start 216.54 86.36) (end 216.4 86.5) (width 0.8) (layer "F.Cu") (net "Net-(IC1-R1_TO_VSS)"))
 (segment (start 216.54 82) (end 216.54 86.36) (width 0.8) (layer "F.Cu") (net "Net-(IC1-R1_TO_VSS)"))
 (segment (start 216.54 111.5) (end 216.54 115.86) (width 0.8) (layer "F.Cu") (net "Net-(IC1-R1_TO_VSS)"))
 (segment (start 216.54 115.86) (end 216.4 116) (width 0.8) (layer "F.Cu") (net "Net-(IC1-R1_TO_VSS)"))
 (segment (start 219.08 86.36) (end 218.94 86.5) (width 0.8) (layer "F.Cu") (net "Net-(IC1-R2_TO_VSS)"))
 (segment (start 219.08 82) (end 219.08 86.36) (width 0.8) (layer "F.Cu") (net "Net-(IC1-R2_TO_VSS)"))
 (segment (start 219.08 115.86) (end 218.94 116) (width 0.8) (layer "F.Cu") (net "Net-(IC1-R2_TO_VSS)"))
 (segment (start 219.08 111.5) (end 219.08 115.86) (width 0.8) (layer "F.Cu") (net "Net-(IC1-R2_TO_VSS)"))
 (segment (start 204.725 82.685) (end 204.725 79.975) (width 0.8) (layer "F.Cu") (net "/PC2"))
 (segment (start 218.845 108.725) (end 221.62 111.5) (width 0.8) (layer "F.Cu") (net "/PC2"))
 (segment (start 221.48 111.64) (end 221.62 111.5) (width 0.8) (layer "F.Cu") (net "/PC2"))
 (segment (start 205.475 108.725) (end 218.845 108.725) (width 0.8) (layer "F.Cu") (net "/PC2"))
 (segment (start 204.725 109.475) (end 205.475 108.725) (width 0.8) (layer "F.Cu") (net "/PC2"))
 (segment (start 221.48 86.5) (end 221.48 82.14) (width 0.8) (layer "F.Cu") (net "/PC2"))
 (segment (start 221.48 82.14) (end 221.62 82) (width 0.8) (layer "F.Cu") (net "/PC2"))
 (segment (start 205.475 79.225) (end 218.845 79.225) (width 0.8) (layer "F.Cu") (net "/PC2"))
 (segment (start 221.48 116) (end 221.48 111.64) (width 0.8) (layer "F.Cu") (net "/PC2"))
 (segment (start 204.725 112.185) (end 204.725 109.475) (width 0.8) (layer "F.Cu") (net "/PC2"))
 (segment (start 218.845 79.225) (end 221.62 82) (width 0.8) (layer "F.Cu") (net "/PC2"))
 (segment (start 204.725 79.975) (end 205.475 79.225) (width 0.8) (layer "F.Cu") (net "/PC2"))
 (segment (start 224.02 111.64) (end 224.16 111.5) (width 0.8) (layer "F.Cu") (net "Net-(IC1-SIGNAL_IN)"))
 (segment (start 224.02 116) (end 224.02 111.64) (width 0.8) (layer "F.Cu") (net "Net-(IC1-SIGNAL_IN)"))
 (segment (start 224.02 82.14) (end 224.16 82) (width 0.8) (layer "F.Cu") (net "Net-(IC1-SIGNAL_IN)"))
 (segment (start 224.02 86.5) (end 224.02 82.14) (width 0.8) (layer "F.Cu") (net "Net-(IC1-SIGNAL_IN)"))
 (segment (start 226.56 111.64) (end 226.7 111.5) (width 0.8) (layer "F.Cu") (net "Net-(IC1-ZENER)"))
 (segment (start 226.56 116) (end 226.56 111.64) (width 0.8) (layer "F.Cu") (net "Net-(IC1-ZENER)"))
 (segment (start 226.56 82.14) (end 226.7 82) (width 0.8) (layer "F.Cu") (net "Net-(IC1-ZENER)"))
 (segment (start 226.56 86.5) (end 226.56 82.14) (width 0.8) (layer "F.Cu") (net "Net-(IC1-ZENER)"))
 (segment (start 229.1 116) (end 229.1 111.64) (width 0.8) (layer "F.Cu") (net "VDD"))
 (segment (start 229.1 82.14) (end 229.24 82) (width 0.8) (layer "F.Cu") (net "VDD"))
 (segment (start 229.1 111.64) (end 229.24 111.5) (width 0.8) (layer "F.Cu") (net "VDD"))
 (segment (start 229.1 86.5) (end 229.1 82.14) (width 0.8) (layer "F.Cu") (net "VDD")))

